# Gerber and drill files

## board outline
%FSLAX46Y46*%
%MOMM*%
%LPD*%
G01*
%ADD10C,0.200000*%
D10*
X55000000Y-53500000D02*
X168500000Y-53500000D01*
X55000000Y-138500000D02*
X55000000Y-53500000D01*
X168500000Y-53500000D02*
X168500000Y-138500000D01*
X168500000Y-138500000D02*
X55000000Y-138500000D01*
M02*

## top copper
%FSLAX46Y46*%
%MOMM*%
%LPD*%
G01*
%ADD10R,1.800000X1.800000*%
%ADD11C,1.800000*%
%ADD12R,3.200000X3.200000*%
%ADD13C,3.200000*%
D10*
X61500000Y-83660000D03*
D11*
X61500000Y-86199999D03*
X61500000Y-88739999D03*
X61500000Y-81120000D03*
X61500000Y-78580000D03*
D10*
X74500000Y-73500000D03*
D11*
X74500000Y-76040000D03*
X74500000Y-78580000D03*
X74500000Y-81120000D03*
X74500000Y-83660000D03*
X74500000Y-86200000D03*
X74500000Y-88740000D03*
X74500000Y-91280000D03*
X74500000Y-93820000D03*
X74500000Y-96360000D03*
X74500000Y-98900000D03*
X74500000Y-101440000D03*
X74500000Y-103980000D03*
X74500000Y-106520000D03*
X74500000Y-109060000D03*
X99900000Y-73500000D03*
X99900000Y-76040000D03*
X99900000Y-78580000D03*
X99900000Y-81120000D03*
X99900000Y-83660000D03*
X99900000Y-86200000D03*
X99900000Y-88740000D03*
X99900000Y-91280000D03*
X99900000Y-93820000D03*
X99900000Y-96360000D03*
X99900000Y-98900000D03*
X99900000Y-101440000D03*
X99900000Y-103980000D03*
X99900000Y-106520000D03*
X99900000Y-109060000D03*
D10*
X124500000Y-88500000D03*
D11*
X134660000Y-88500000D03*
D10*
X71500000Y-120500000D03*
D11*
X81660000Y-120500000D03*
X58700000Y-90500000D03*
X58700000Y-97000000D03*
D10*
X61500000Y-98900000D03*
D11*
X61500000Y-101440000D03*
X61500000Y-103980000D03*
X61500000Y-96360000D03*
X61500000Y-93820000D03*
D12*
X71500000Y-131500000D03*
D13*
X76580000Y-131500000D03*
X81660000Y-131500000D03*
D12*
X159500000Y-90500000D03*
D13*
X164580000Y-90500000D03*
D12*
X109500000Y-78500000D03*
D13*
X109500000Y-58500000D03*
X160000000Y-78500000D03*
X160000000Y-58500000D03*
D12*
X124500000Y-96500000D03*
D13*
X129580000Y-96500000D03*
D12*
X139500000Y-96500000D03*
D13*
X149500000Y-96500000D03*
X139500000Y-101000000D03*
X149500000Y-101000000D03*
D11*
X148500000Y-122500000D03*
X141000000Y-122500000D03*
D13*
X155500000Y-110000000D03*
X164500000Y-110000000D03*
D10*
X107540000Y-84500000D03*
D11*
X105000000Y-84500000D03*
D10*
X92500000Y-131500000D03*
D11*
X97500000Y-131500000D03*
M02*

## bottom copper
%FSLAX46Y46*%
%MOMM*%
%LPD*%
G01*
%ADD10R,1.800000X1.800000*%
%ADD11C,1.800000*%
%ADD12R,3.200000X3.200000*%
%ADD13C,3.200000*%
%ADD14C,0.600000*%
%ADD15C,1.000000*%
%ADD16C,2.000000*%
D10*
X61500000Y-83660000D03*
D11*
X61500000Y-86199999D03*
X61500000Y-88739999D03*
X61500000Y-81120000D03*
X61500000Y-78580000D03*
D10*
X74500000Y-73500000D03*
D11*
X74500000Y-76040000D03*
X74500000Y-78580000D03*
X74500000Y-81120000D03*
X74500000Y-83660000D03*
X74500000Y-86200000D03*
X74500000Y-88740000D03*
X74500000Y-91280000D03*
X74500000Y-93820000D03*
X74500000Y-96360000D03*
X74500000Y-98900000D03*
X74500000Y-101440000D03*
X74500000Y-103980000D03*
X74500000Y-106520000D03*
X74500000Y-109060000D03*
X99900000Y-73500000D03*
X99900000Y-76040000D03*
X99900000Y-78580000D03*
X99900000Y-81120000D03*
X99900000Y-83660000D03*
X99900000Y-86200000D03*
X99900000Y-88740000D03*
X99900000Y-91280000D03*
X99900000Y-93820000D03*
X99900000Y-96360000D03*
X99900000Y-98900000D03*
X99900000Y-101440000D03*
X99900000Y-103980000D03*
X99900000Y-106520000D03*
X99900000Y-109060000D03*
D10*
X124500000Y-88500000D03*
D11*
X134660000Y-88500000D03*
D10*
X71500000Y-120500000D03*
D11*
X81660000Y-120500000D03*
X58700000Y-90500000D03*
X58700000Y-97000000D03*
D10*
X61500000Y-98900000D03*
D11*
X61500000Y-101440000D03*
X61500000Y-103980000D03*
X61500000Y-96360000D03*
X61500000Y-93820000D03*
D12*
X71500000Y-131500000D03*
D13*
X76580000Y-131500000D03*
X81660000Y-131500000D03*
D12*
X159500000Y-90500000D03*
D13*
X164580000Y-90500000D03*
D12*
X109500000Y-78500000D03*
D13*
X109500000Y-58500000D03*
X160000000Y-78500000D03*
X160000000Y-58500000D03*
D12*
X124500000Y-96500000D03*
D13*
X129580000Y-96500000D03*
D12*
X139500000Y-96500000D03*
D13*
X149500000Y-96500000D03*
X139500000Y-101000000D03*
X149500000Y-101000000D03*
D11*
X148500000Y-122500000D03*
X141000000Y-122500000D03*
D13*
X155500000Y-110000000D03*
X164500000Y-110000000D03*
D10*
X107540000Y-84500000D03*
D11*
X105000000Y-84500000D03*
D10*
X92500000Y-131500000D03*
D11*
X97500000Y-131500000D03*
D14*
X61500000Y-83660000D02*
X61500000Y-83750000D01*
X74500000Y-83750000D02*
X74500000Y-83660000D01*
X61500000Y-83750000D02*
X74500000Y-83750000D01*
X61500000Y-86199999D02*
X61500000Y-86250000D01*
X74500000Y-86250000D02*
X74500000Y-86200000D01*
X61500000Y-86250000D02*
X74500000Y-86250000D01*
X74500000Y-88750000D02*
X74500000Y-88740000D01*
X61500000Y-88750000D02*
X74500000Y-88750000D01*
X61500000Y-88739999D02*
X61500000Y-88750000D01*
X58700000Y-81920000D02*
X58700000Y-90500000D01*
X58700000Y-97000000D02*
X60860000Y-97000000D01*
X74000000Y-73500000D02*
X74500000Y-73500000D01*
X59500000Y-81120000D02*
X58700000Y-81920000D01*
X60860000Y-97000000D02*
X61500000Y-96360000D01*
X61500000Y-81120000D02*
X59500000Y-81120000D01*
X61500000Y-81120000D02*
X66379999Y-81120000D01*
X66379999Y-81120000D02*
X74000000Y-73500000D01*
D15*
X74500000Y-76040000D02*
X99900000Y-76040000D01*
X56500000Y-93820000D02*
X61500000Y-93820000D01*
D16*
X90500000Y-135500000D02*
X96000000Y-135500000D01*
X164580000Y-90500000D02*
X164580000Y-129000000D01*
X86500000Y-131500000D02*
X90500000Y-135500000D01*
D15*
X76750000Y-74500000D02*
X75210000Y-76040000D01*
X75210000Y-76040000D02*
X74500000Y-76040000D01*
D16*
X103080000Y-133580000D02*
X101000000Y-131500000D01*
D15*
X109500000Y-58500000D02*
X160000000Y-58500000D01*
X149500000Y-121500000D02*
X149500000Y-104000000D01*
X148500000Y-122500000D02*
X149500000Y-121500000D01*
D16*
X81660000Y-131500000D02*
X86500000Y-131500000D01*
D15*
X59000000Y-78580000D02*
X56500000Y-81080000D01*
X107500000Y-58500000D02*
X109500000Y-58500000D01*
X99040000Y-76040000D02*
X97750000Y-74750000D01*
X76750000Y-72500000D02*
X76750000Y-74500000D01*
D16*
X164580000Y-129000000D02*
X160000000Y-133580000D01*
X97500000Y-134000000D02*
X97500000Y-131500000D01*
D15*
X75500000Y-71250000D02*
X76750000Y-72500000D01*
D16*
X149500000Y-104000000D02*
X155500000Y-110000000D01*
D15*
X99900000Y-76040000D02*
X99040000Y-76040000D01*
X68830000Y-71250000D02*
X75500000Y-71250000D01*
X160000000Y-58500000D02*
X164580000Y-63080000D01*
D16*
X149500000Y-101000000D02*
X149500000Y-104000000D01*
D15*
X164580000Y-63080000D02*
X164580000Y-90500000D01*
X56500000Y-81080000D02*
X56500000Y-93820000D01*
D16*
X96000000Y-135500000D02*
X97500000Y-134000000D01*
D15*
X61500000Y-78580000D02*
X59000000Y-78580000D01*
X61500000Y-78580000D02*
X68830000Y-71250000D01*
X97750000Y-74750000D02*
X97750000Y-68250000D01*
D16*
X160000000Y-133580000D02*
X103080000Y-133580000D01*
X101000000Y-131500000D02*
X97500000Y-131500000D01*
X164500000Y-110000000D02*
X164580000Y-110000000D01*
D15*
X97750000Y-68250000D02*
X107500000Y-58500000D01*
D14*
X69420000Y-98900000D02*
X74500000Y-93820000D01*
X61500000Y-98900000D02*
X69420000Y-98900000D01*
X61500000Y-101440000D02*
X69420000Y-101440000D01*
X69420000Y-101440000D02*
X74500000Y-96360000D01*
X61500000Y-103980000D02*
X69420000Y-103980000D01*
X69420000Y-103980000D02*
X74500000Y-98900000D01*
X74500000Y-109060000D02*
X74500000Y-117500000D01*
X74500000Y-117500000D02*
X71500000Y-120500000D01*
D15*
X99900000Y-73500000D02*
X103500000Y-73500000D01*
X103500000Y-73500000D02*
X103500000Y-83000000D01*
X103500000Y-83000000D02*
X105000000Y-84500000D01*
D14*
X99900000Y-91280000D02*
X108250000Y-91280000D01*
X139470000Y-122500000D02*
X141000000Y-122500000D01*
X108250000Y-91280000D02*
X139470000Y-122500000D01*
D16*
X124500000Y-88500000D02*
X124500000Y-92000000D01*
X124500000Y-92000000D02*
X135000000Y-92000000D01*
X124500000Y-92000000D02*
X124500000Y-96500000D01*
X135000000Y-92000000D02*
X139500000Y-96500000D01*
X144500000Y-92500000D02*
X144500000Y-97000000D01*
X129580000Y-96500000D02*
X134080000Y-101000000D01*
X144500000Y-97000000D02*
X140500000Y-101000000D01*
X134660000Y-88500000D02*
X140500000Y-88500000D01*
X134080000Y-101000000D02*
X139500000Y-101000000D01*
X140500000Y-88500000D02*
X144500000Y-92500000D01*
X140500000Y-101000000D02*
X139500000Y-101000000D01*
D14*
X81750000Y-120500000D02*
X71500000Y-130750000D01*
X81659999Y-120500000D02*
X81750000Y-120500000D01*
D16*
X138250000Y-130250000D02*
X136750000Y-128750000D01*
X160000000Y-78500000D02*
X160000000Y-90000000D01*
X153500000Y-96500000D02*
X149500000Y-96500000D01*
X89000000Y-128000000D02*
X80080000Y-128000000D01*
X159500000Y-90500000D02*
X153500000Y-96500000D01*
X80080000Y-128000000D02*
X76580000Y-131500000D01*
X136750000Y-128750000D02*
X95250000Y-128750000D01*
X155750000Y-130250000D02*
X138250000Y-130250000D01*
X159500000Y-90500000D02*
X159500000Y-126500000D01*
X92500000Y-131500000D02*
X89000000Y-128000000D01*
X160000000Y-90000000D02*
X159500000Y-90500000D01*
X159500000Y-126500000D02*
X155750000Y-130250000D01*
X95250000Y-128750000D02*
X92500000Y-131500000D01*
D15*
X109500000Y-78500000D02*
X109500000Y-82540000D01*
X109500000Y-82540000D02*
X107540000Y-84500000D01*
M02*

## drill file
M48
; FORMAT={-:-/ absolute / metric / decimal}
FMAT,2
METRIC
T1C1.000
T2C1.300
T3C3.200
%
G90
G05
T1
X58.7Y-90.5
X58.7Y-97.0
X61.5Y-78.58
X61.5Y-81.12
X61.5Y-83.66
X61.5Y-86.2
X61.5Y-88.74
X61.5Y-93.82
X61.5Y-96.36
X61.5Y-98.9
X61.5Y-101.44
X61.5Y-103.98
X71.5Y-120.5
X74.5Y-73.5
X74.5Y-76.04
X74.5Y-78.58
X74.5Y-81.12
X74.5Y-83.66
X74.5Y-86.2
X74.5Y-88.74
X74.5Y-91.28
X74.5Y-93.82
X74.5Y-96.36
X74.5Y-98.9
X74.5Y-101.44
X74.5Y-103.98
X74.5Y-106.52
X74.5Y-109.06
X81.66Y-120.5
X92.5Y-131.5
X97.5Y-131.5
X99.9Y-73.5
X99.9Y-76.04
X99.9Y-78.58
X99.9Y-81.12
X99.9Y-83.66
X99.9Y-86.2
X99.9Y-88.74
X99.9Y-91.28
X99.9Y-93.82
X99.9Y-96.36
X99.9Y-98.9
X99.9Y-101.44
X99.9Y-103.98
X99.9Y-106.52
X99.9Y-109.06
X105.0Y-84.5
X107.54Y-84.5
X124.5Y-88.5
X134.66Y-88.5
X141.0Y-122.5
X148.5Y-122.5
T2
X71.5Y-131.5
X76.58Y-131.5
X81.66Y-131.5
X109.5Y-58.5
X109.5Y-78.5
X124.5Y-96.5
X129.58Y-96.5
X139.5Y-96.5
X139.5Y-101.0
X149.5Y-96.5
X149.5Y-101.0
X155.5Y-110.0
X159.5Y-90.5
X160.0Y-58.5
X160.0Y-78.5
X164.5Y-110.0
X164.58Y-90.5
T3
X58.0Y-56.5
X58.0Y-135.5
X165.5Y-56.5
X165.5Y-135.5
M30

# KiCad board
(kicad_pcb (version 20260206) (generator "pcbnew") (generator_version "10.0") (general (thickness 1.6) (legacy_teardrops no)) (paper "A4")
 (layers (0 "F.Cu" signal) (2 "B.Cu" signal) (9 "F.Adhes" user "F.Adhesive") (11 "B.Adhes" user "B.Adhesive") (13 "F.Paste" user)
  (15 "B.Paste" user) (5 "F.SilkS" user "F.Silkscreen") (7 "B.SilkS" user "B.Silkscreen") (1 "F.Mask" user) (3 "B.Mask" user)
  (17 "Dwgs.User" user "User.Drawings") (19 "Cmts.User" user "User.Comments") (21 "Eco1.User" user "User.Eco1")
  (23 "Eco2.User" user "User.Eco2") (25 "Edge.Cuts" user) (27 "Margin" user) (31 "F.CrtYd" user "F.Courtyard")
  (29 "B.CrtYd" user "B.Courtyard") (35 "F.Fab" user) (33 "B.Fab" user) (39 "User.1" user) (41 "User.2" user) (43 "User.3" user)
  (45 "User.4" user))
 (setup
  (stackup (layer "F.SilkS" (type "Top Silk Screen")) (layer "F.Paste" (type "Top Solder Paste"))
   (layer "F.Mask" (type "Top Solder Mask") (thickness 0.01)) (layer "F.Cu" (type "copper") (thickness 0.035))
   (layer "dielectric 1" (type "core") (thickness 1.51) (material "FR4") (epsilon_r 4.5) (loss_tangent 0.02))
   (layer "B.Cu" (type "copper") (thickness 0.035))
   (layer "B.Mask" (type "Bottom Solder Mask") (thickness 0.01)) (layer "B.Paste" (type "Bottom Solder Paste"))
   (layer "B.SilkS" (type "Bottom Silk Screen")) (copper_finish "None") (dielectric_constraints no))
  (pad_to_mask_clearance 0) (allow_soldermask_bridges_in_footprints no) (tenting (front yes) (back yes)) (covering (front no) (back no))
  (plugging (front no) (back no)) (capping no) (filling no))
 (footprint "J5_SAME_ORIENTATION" (layer "F.Cu") (at 61.5 83.5 -90)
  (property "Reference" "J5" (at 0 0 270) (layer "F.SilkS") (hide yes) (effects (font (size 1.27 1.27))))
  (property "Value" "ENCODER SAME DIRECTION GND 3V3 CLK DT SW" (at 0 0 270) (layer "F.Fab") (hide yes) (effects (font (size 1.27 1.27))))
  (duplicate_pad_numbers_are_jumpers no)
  (pad "1" thru_hole rect (at 0.16 0 270) (size 1.8 1.8) (drill 1) (layers "*.Cu") (remove_unused_layers no) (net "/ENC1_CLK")
   (clearance 0.5) (thermal_bridge_angle 45))
  (pad "2" thru_hole circle (at 2.699999 0 270) (size 1.8 1.8) (drill 1) (layers "*.Cu") (remove_unused_layers no) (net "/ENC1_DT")
   (clearance 0.5))
  (pad "3" thru_hole circle (at 5.239999 0 270) (size 1.8 1.8) (drill 1) (layers "*.Cu") (remove_unused_layers no) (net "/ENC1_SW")
   (clearance 0.5))
  (pad "4" thru_hole circle (at -2.38 0 270) (size 1.8 1.8) (drill 1) (layers "*.Cu") (remove_unused_layers no) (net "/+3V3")
   (clearance 0.5))
  (pad "5" thru_hole circle (at -4.92 0 270) (size 1.8 1.8) (drill 1) (layers "*.Cu") (remove_unused_layers no) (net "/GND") (clearance 0.5)))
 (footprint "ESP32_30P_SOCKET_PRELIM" (layer "F.Cu") (at 74.5 73.5)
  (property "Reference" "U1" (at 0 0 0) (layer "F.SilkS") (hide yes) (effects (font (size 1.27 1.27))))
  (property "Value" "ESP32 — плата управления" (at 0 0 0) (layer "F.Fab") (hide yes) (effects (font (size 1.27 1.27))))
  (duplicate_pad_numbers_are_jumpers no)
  (pad "1" thru_hole rect (at 0 0) (size 1.8 1.8) (drill 1) (layers "*.Cu") (remove_unused_layers no) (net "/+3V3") (clearance 0.5)
   (thermal_bridge_angle 45))
  (pad "2" thru_hole circle (at 0 2.54) (size 1.8 1.8) (drill 1) (layers "*.Cu") (remove_unused_layers no) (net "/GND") (clearance 0.5))
  (pad "3" thru_hole circle (at 0 5.08) (size 1.8 1.8) (drill 1) (layers "*.Cu") (remove_unused_layers no) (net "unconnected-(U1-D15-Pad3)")
   (clearance 0.5))
  (pad "4" thru_hole circle (at 0 7.62) (size 1.8 1.8) (drill 1) (layers "*.Cu") (remove_unused_layers no) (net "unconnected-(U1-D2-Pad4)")
   (clearance 0.5))
  (pad "5" thru_hole circle (at 0 10.16) (size 1.8 1.8) (drill 1) (layers "*.Cu") (remove_unused_layers no) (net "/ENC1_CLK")
   (clearance 0.5))
  (pad "6" thru_hole circle (at 0 12.7) (size 1.8 1.8) (drill 1) (layers "*.Cu") (remove_unused_layers no) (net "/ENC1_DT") (clearance 0.5))
  (pad "7" thru_hole circle (at 0 15.24) (size 1.8 1.8) (drill 1) (layers "*.Cu") (remove_unused_layers no) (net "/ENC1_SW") (clearance 0.5))
  (pad "8" thru_hole circle (at 0 17.78) (size 1.8 1.8) (drill 1) (layers "*.Cu") (remove_unused_layers no) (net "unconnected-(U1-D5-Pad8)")
   (clearance 0.5))
  (pad "9" thru_hole circle (at 0 20.32) (size 1.8 1.8) (drill 1) (layers "*.Cu") (remove_unused_layers no) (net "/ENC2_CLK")
   (clearance 0.5))
  (pad "10" thru_hole circle (at 0 22.86) (size 1.8 1.8) (drill 1) (layers "*.Cu") (remove_unused_layers no) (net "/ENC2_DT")
   (clearance 0.5))
  (pad "11" thru_hole circle (at 0 25.4) (size 1.8 1.8) (drill 1) (layers "*.Cu") (remove_unused_layers no) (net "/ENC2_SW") (clearance 0.5))
  (pad "12" thru_hole circle (at 0 27.94) (size 1.8 1.8) (drill 1) (layers "*.Cu") (remove_unused_layers no)
   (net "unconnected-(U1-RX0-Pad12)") (clearance 0.5))
  (pad "13" thru_hole circle (at 0 30.48) (size 1.8 1.8) (drill 1) (layers "*.Cu") (remove_unused_layers no)
   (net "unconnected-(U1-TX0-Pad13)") (clearance 0.5))
  (pad "14" thru_hole circle (at 0 33.02) (size 1.8 1.8) (drill 1) (layers "*.Cu") (remove_unused_layers no)
   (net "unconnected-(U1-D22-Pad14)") (clearance 0.5))
  (pad "15" thru_hole circle (at 0 35.56) (size 1.8 1.8) (drill 1) (layers "*.Cu") (remove_unused_layers no) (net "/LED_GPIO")
   (clearance 0.5))
  (pad "16" thru_hole circle (at 25.4 0) (size 1.8 1.8) (drill 1) (layers "*.Cu") (remove_unused_layers no) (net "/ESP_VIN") (clearance 0.5))
  (pad "17" thru_hole circle (at 25.4 2.54) (size 1.8 1.8) (drill 1) (layers "*.Cu") (remove_unused_layers no) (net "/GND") (clearance 0.5))
  (pad "18" thru_hole circle (at 25.4 5.08) (size 1.8 1.8) (drill 1) (layers "*.Cu") (remove_unused_layers no)
   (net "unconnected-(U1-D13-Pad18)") (clearance 0.5))
  (pad "19" thru_hole circle (at 25.4 7.62) (size 1.8 1.8) (drill 1) (layers "*.Cu") (remove_unused_layers no)
   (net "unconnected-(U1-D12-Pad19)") (clearance 0.5))
  (pad "20" thru_hole circle (at 25.4 10.16) (size 1.8 1.8) (drill 1) (layers "*.Cu") (remove_unused_layers no)
   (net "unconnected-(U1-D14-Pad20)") (clearance 0.5))
  (pad "21" thru_hole circle (at 25.4 12.7) (size 1.8 1.8) (drill 1) (layers "*.Cu") (remove_unused_layers no)
   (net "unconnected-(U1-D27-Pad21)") (clearance 0.5))
  (pad "22" thru_hole circle (at 25.4 15.24) (size 1.8 1.8) (drill 1) (layers "*.Cu") (remove_unused_layers no)
   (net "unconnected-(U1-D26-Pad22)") (clearance 0.5))
  (pad "23" thru_hole circle (at 25.4 17.78) (size 1.8 1.8) (drill 1) (layers "*.Cu") (remove_unused_layers no) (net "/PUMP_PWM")
   (clearance 0.5))
  (pad "24" thru_hole circle (at 25.4 20.32) (size 1.8 1.8) (drill 1) (layers "*.Cu") (remove_unused_layers no)
   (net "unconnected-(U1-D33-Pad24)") (clearance 0.5))
  (pad "25" thru_hole circle (at 25.4 22.86) (size 1.8 1.8) (drill 1) (layers "*.Cu") (remove_unused_layers no)
   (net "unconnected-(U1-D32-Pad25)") (clearance 0.5))
  (pad "26" thru_hole circle (at 25.4 25.4) (size 1.8 1.8) (drill 1) (layers "*.Cu") (remove_unused_layers no)
   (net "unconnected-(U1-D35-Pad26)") (clearance 0.5))
  (pad "27" thru_hole circle (at 25.4 27.94) (size 1.8 1.8) (drill 1) (layers "*.Cu") (remove_unused_layers no)
   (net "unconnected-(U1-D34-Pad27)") (clearance 0.5))
  (pad "28" thru_hole circle (at 25.4 30.48) (size 1.8 1.8) (drill 1) (layers "*.Cu") (remove_unused_layers no)
   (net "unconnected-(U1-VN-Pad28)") (clearance 0.5))
  (pad "29" thru_hole circle (at 25.4 33.02) (size 1.8 1.8) (drill 1) (layers "*.Cu") (remove_unused_layers no)
   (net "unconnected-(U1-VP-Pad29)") (clearance 0.5))
  (pad "30" thru_hole circle (at 25.4 35.56) (size 1.8 1.8) (drill 1) (layers "*.Cu") (remove_unused_layers no)
   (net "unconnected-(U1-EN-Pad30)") (clearance 0.5)))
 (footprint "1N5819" (layer "F.Cu") (at 124.5 88.5)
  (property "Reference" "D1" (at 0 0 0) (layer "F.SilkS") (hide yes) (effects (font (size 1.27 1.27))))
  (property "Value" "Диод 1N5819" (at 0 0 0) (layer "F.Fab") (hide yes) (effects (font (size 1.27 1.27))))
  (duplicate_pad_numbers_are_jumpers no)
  (pad "1" thru_hole rect (at 0 0) (size 1.8 1.8) (drill 1) (layers "*.Cu") (remove_unused_layers no) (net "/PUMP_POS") (clearance 0.5)
   (thermal_bridge_angle 45))
  (pad "2" thru_hole circle (at 10.16 0) (size 1.8 1.8) (drill 1) (layers "*.Cu") (remove_unused_layers no) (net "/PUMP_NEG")
   (clearance 0.5)))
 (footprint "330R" (layer "F.Cu") (at 71.5 120.5)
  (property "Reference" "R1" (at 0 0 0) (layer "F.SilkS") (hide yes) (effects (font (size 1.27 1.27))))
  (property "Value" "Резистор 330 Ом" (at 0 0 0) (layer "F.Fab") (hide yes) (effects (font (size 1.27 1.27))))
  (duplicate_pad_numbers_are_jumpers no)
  (pad "1" thru_hole rect (at 0 0) (size 1.8 1.8) (drill 1) (layers "*.Cu") (remove_unused_layers no) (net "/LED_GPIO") (clearance 0.5)
   (thermal_bridge_angle 45))
  (pad "2" thru_hole circle (at 10.16 0) (size 1.8 1.8) (drill 1) (layers "*.Cu") (remove_unused_layers no) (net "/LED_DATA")
   (clearance 0.5)))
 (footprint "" (layer "F.Cu") (at 58 135.5)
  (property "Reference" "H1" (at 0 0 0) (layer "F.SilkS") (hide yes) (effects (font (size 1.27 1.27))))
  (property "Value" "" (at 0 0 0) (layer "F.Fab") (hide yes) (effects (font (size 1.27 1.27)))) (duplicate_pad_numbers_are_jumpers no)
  (pad "" np_thru_hole circle (at 0 0) (size 3.2 3.2) (drill 3.2) (layers "*.Cu") (clearance 0.5)))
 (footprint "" (layer "F.Cu") (at 58.7 90.5)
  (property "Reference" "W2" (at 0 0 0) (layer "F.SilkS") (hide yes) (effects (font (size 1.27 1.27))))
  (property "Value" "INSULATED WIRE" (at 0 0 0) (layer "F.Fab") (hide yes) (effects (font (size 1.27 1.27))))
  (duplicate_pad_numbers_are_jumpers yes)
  (pad "1" thru_hole circle (at 0 0) (size 1.8 1.8) (drill 1) (layers "*.Cu") (remove_unused_layers no) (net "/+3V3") (clearance 0.5))
  (pad "1" thru_hole circle (at 0 6.5) (size 1.8 1.8) (drill 1) (layers "*.Cu") (remove_unused_layers no) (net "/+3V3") (clearance 0.5)))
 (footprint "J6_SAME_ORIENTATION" (layer "F.Cu") (at 61.5 96.5 -90)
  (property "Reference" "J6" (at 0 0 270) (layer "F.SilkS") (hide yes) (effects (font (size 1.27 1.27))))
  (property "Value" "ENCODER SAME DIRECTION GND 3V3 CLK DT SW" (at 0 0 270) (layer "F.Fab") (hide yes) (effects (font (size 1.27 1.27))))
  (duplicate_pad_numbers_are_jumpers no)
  (pad "1" thru_hole rect (at 2.4 0 270) (size 1.8 1.8) (drill 1) (layers "*.Cu") (remove_unused_layers no) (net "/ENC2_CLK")
   (clearance 0.5) (thermal_bridge_angle 45))
  (pad "2" thru_hole circle (at 4.94 0 270) (size 1.8 1.8) (drill 1) (layers "*.Cu") (remove_unused_layers no) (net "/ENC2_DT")
   (clearance 0.5))
  (pad "3" thru_hole circle (at 7.48 0 270) (size 1.8 1.8) (drill 1) (layers "*.Cu") (remove_unused_layers no) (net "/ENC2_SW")
   (clearance 0.5))
  (pad "4" thru_hole circle (at -0.14 0 270) (size 1.8 1.8) (drill 1) (layers "*.Cu") (remove_unused_layers no) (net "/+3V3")
   (clearance 0.5))
  (pad "5" thru_hole circle (at -2.68 0 270) (size 1.8 1.8) (drill 1) (layers "*.Cu") (remove_unused_layers no) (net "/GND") (clearance 0.5)))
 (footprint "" (layer "F.Cu") (at 58 56.5)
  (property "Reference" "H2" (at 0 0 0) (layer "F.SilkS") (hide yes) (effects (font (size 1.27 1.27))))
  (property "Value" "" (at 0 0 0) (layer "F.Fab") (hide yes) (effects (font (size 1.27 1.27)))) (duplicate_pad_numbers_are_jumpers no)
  (pad "" np_thru_hole circle (at 0 0) (size 3.2 3.2) (drill 3.2) (layers "*.Cu") (clearance 0.5)))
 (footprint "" (layer "F.Cu") (at 165.5 135.5)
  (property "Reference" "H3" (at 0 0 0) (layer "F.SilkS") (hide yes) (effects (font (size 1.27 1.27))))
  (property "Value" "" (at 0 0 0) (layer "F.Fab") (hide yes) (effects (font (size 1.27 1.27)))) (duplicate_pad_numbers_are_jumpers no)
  (pad "" np_thru_hole circle (at 0 0) (size 3.2 3.2) (drill 3.2) (layers "*.Cu") (clearance 0.5)))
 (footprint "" (layer "F.Cu") (at 165.5 56.5)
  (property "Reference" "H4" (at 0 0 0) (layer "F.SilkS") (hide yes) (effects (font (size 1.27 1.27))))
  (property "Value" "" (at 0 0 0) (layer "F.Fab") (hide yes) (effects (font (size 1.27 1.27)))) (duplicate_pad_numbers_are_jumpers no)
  (pad "" np_thru_hole circle (at 0 0) (size 3.2 3.2) (drill 3.2) (layers "*.Cu") (clearance 0.5)))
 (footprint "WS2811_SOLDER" (layer "F.Cu") (at 71.5 131.5)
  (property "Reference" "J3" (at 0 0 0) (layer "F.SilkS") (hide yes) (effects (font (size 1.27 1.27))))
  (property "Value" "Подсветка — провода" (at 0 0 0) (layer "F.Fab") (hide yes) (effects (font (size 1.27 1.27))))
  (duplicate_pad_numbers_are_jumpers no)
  (pad "1" thru_hole rect (at 0 0) (size 3.2 3.2) (drill 1.3) (layers "*.Cu") (remove_unused_layers no) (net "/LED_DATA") (clearance 0.5)
   (thermal_bridge_angle 45))
  (pad "2" thru_hole circle (at 5.08 0) (size 3.2 3.2) (drill 1.3) (layers "*.Cu") (remove_unused_layers no) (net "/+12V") (clearance 0.5))
  (pad "3" thru_hole circle (at 10.16 0) (size 3.2 3.2) (drill 1.3) (layers "*.Cu") (remove_unused_layers no) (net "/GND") (clearance 0.5)))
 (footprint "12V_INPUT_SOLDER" (layer "F.Cu") (at 159.5 90.5)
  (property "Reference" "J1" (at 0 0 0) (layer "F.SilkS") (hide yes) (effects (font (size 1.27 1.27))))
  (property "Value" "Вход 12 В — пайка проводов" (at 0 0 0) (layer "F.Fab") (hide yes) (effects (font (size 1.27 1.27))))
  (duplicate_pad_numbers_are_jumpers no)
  (pad "1" thru_hole rect (at 0 0) (size 3.2 3.2) (drill 1.3) (layers "*.Cu") (remove_unused_layers no) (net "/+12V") (clearance 0.5)
   (thermal_bridge_angle 45))
  (pad "2" thru_hole circle (at 5.08 0) (size 3.2 3.2) (drill 1.3) (layers "*.Cu") (remove_unused_layers no) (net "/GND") (clearance 0.5)))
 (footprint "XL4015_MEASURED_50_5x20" (layer "F.Cu") (at 109.5 78.5 90)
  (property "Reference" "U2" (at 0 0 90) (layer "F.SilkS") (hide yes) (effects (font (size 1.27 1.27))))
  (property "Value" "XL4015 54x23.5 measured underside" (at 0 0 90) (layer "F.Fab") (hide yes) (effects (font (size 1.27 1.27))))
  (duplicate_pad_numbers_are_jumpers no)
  (pad "1" thru_hole rect (at 0 0 90) (size 3.2 3.2) (drill 1.3) (layers "*.Cu") (remove_unused_layers no) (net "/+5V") (clearance 0.5)
   (thermal_bridge_angle 45))
  (pad "2" thru_hole circle (at 20 0 90) (size 3.2 3.2) (drill 1.3) (layers "*.Cu") (remove_unused_layers no) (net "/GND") (clearance 0.5))
  (pad "3" thru_hole circle (at 0 50.5 90) (size 3.2 3.2) (drill 1.3) (layers "*.Cu") (remove_unused_layers no) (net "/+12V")
   (clearance 0.5))
  (pad "4" thru_hole circle (at 20 50.5 90) (size 3.2 3.2) (drill 1.3) (layers "*.Cu") (remove_unused_layers no) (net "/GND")
   (clearance 0.5)))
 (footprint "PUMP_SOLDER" (layer "F.Cu") (at 124.5 96.5)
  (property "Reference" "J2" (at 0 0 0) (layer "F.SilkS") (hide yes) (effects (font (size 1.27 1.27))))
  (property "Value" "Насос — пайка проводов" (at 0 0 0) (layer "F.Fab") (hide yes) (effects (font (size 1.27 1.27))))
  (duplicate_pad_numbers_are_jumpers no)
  (pad "1" thru_hole rect (at 0 0) (size 3.2 3.2) (drill 1.3) (layers "*.Cu") (remove_unused_layers no) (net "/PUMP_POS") (clearance 0.5)
   (thermal_bridge_angle 45))
  (pad "2" thru_hole circle (at 5.08 0) (size 3.2 3.2) (drill 1.3) (layers "*.Cu") (remove_unused_layers no) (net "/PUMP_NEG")
   (clearance 0.5)))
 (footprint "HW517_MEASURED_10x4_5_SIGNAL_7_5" (layer "F.Cu") (at 139.5 96.5)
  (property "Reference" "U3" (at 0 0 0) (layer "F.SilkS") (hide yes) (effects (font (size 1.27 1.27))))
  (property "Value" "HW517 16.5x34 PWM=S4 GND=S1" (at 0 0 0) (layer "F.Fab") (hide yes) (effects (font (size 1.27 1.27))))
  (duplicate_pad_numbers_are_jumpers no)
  (pad "1" thru_hole rect (at 0 0) (size 3.2 3.2) (drill 1.3) (layers "*.Cu") (remove_unused_layers no) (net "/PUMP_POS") (clearance 0.5)
   (thermal_bridge_angle 45))
  (pad "2" thru_hole circle (at 10 0) (size 3.2 3.2) (drill 1.3) (layers "*.Cu") (remove_unused_layers no) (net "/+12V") (clearance 0.5))
  (pad "3" thru_hole circle (at 0 4.5) (size 3.2 3.2) (drill 1.3) (layers "*.Cu") (remove_unused_layers no) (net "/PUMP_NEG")
   (clearance 0.5))
  (pad "4" thru_hole circle (at 10 4.5) (size 3.2 3.2) (drill 1.3) (layers "*.Cu") (remove_unused_layers no) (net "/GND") (clearance 0.5))
  (pad "5" thru_hole circle (at 9 26) (size 1.8 1.8) (drill 1) (layers "*.Cu") (remove_unused_layers no) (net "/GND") (clearance 0.5))
  (pad "6" thru_hole circle (at 1.5 26) (size 1.8 1.8) (drill 1) (layers "*.Cu") (remove_unused_layers no) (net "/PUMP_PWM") (clearance 0.5)))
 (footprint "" (layer "F.Cu") (at 155.5 110)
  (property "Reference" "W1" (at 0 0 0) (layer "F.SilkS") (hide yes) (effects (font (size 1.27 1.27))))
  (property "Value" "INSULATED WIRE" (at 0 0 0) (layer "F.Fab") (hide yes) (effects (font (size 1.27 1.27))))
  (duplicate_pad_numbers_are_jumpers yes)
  (pad "1" thru_hole circle (at 0 0) (size 3.2 3.2) (drill 1.3) (layers "*.Cu") (remove_unused_layers no) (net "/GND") (clearance 0.5))
  (pad "1" thru_hole circle (at 9 0) (size 3.2 3.2) (drill 1.3) (layers "*.Cu") (remove_unused_layers no) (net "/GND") (clearance 0.5)))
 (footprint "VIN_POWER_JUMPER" (layer "F.Cu") (at 107.54 84.5)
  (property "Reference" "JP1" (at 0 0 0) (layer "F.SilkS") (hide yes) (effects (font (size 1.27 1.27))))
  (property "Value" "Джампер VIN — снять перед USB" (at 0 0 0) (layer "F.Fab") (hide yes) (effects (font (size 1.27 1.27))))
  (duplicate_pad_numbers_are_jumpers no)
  (pad "1" thru_hole rect (at 0 0) (size 1.8 1.8) (drill 1) (layers "*.Cu") (remove_unused_layers no) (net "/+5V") (clearance 0.5)
   (thermal_bridge_angle 45))
  (pad "2" thru_hole circle (at -2.54 0) (size 1.8 1.8) (drill 1) (layers "*.Cu") (remove_unused_layers no) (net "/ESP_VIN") (clearance 0.5)))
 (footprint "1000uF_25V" (layer "F.Cu") (at 92.5 131.5)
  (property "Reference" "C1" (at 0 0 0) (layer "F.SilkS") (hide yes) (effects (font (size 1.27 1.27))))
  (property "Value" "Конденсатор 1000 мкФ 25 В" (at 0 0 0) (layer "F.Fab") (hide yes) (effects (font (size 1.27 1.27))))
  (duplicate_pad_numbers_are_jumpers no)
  (pad "1" thru_hole rect (at 0 0) (size 1.8 1.8) (drill 1) (layers "*.Cu") (remove_unused_layers no) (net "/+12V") (clearance 0.5)
   (thermal_bridge_angle 45))
  (pad "2" thru_hole circle (at 5 0) (size 1.8 1.8) (drill 1) (layers "*.Cu") (remove_unused_layers no) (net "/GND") (clearance 0.5)))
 (gr_line (start 55 53.5) (end 168.5 53.5) (stroke (width 0.2) (type default)) (layer "Edge.Cuts"))
 (gr_line (start 55 138.5) (end 55 53.5) (stroke (width 0.2) (type default)) (layer "Edge.Cuts"))
 (gr_line (start 168.5 53.5) (end 168.5 138.5) (stroke (width 0.2) (type default)) (layer "Edge.Cuts"))
 (gr_line (start 168.5 138.5) (end 55 138.5) (stroke (width 0.2) (type default)) (layer "Edge.Cuts"))
 (segment (start 61.5 83.66) (end 61.5 83.75) (width 0.6) (layer "B.Cu") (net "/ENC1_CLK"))
 (segment (start 74.5 83.75) (end 74.5 83.66) (width 0.6) (layer "B.Cu") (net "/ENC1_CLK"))
 (segment (start 61.5 83.75) (end 74.5 83.75) (width 0.6) (layer "B.Cu") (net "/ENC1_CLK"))
 (segment (start 61.5 86.199999) (end 61.5 86.25) (width 0.6) (layer "B.Cu") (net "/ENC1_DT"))
 (segment (start 74.5 86.25) (end 74.5 86.2) (width 0.6) (layer "B.Cu") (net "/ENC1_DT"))
 (segment (start 61.5 86.25) (end 74.5 86.25) (width 0.6) (layer "B.Cu") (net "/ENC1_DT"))
 (segment (start 74.5 88.75) (end 74.5 88.74) (width 0.6) (layer "B.Cu") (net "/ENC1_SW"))
 (segment (start 61.5 88.75) (end 74.5 88.75) (width 0.6) (layer "B.Cu") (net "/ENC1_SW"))
 (segment (start 61.5 88.739999) (end 61.5 88.75) (width 0.6) (layer "B.Cu") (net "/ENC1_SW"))
 (segment (start 58.7 81.92) (end 58.7 90.5) (width 0.6) (layer "B.Cu") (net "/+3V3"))
 (segment (start 58.7 97) (end 60.86 97) (width 0.6) (layer "B.Cu") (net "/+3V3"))
 (segment (start 74 73.5) (end 74.5 73.5) (width 0.6) (layer "B.Cu") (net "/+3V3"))
 (segment (start 59.5 81.12) (end 58.7 81.92) (width 0.6) (layer "B.Cu") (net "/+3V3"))
 (segment (start 60.86 97) (end 61.5 96.36) (width 0.6) (layer "B.Cu") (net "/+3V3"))
 (segment (start 61.5 81.12) (end 59.5 81.12) (width 0.6) (layer "B.Cu") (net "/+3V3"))
 (segment (start 61.5 81.12) (end 66.379999 81.12) (width 0.6) (layer "B.Cu") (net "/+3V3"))
 (segment (start 66.379999 81.12) (end 74 73.5) (width 0.6) (layer "B.Cu") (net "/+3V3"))
 (segment (start 74.5 76.04) (end 99.9 76.04) (width 1) (layer "B.Cu") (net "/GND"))
 (segment (start 56.5 93.82) (end 61.5 93.82) (width 1) (layer "B.Cu") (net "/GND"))
 (segment (start 90.5 135.5) (end 96 135.5) (width 2) (layer "B.Cu") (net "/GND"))
 (segment (start 164.58 90.5) (end 164.58 129) (width 2) (layer "B.Cu") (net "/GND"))
 (segment (start 86.5 131.5) (end 90.5 135.5) (width 2) (layer "B.Cu") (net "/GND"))
 (segment (start 76.75 74.5) (end 75.21 76.04) (width 1) (layer "B.Cu") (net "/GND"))
 (segment (start 75.21 76.04) (end 74.5 76.04) (width 1) (layer "B.Cu") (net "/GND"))
 (segment (start 103.08 133.58) (end 101 131.5) (width 2) (layer "B.Cu") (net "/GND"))
 (segment (start 109.5 58.5) (end 160 58.5) (width 1) (layer "B.Cu") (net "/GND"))
 (segment (start 149.5 121.5) (end 149.5 104) (width 1) (layer "B.Cu") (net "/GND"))
 (segment (start 148.5 122.5) (end 149.5 121.5) (width 1) (layer "B.Cu") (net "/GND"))
 (segment (start 81.66 131.5) (end 86.5 131.5) (width 2) (layer "B.Cu") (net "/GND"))
 (segment (start 59 78.58) (end 56.5 81.08) (width 1) (layer "B.Cu") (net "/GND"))
 (segment (start 107.5 58.5) (end 109.5 58.5) (width 1) (layer "B.Cu") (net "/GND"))
 (segment (start 99.04 76.04) (end 97.75 74.75) (width 1) (layer "B.Cu") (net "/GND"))
 (segment (start 76.75 72.5) (end 76.75 74.5) (width 1) (layer "B.Cu") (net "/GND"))
 (segment (start 164.58 129) (end 160 133.58) (width 2) (layer "B.Cu") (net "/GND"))
 (segment (start 97.5 134) (end 97.5 131.5) (width 2) (layer "B.Cu") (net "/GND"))
 (segment (start 75.5 71.25) (end 76.75 72.5) (width 1) (layer "B.Cu") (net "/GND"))
 (segment (start 149.5 104) (end 155.5 110) (width 2) (layer "B.Cu") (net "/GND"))
 (segment (start 99.9 76.04) (end 99.04 76.04) (width 1) (layer "B.Cu") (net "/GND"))
 (segment (start 68.83 71.25) (end 75.5 71.25) (width 1) (layer "B.Cu") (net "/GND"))
 (segment (start 160 58.5) (end 164.58 63.08) (width 1) (layer "B.Cu") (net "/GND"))
 (segment (start 149.5 101) (end 149.5 104) (width 2) (layer "B.Cu") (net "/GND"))
 (segment (start 164.58 63.08) (end 164.58 90.5) (width 1) (layer "B.Cu") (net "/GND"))
 (segment (start 56.5 81.08) (end 56.5 93.82) (width 1) (layer "B.Cu") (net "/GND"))
 (segment (start 96 135.5) (end 97.5 134) (width 2) (layer "B.Cu") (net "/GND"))
 (segment (start 61.5 78.58) (end 59 78.58) (width 1) (layer "B.Cu") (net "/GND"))
 (segment (start 61.5 78.58) (end 68.83 71.25) (width 1) (layer "B.Cu") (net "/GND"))
 (segment (start 97.75 74.75) (end 97.75 68.25) (width 1) (layer "B.Cu") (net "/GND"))
 (segment (start 160 133.58) (end 103.08 133.58) (width 2) (layer "B.Cu") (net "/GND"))
 (segment (start 101 131.5) (end 97.5 131.5) (width 2) (layer "B.Cu") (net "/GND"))
 (segment (start 164.5 110) (end 164.58 110) (width 2) (layer "B.Cu") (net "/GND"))
 (segment (start 97.75 68.25) (end 107.5 58.5) (width 1) (layer "B.Cu") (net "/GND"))
 (segment (start 69.42 98.9) (end 74.5 93.82) (width 0.6) (layer "B.Cu") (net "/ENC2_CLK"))
 (segment (start 61.5 98.9) (end 69.42 98.9) (width 0.6) (layer "B.Cu") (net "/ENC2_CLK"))
 (segment (start 61.5 101.44) (end 69.42 101.44) (width 0.6) (layer "B.Cu") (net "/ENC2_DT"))
 (segment (start 69.42 101.44) (end 74.5 96.36) (width 0.6) (layer "B.Cu") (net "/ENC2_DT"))
 (segment (start 61.5 103.98) (end 69.42 103.98) (width 0.6) (layer "B.Cu") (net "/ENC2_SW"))
 (segment (start 69.42 103.98) (end 74.5 98.9) (width 0.6) (layer "B.Cu") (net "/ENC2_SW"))
 (segment (start 74.5 109.06) (end 74.5 117.5) (width 0.6) (layer "B.Cu") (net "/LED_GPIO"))
 (segment (start 74.5 117.5) (end 71.5 120.5) (width 0.6) (layer "B.Cu") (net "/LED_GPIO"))
 (segment (start 99.9 73.5) (end 103.5 73.5) (width 1) (layer "B.Cu") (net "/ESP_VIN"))
 (segment (start 103.5 73.5) (end 103.5 83) (width 1) (layer "B.Cu") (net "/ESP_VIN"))
 (segment (start 103.5 83) (end 105 84.5) (width 1) (layer "B.Cu") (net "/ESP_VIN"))
 (segment (start 99.9 91.28) (end 108.25 91.28) (width 0.6) (layer "B.Cu") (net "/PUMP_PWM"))
 (segment (start 139.47 122.5) (end 141 122.5) (width 0.6) (layer "B.Cu") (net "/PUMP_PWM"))
 (segment (start 108.25 91.28) (end 139.47 122.5) (width 0.6) (layer "B.Cu") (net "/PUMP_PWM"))
 (segment (start 124.5 88.5) (end 124.5 92) (width 2) (layer "B.Cu") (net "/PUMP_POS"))
 (segment (start 124.5 92) (end 135 92) (width 2) (layer "B.Cu") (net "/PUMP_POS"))
 (segment (start 124.5 92) (end 124.5 96.5) (width 2) (layer "B.Cu") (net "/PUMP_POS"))
 (segment (start 135 92) (end 139.5 96.5) (width 2) (layer "B.Cu") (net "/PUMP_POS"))
 (segment (start 144.5 92.5) (end 144.5 97) (width 2) (layer "B.Cu") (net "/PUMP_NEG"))
 (segment (start 129.58 96.5) (end 134.08 101) (width 2) (layer "B.Cu") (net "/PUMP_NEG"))
 (segment (start 144.5 97) (end 140.5 101) (width 2) (layer "B.Cu") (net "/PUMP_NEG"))
 (segment (start 134.66 88.5) (end 140.5 88.5) (width 2) (layer "B.Cu") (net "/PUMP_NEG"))
 (segment (start 134.08 101) (end 139.5 101) (width 2) (layer "B.Cu") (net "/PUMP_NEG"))
 (segment (start 140.5 88.5) (end 144.5 92.5) (width 2) (layer "B.Cu") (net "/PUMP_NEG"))
 (segment (start 140.5 101) (end 139.5 101) (width 2) (layer "B.Cu") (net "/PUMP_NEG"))
 (segment (start 81.75 120.5) (end 71.5 130.75) (width 0.6) (layer "B.Cu") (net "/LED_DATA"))
 (segment (start 81.659999 120.5) (end 81.75 120.5) (width 0.6) (layer "B.Cu") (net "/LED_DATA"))
 (segment (start 138.25 130.25) (end 136.75 128.75) (width 2) (layer "B.Cu") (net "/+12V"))
 (segment (start 160 78.5) (end 160 90) (width 2) (layer "B.Cu") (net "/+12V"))
 (segment (start 153.5 96.5) (end 149.5 96.5) (width 2) (layer "B.Cu") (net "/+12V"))
 (segment (start 89 128) (end 80.08 128) (width 2) (layer "B.Cu") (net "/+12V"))
 (segment (start 159.5 90.5) (end 153.5 96.5) (width 2) (layer "B.Cu") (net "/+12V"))
 (segment (start 80.08 128) (end 76.58 131.5) (width 2) (layer "B.Cu") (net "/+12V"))
 (segment (start 136.75 128.75) (end 95.25 128.75) (width 2) (layer "B.Cu") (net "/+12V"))
 (segment (start 155.75 130.25) (end 138.25 130.25) (width 2) (layer "B.Cu") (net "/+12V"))
 (segment (start 159.5 90.5) (end 159.5 126.5) (width 2) (layer "B.Cu") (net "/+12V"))
 (segment (start 92.5 131.5) (end 89 128) (width 2) (layer "B.Cu") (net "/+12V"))
 (segment (start 160 90) (end 159.5 90.5) (width 2) (layer "B.Cu") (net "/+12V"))
 (segment (start 159.5 126.5) (end 155.75 130.25) (width 2) (layer "B.Cu") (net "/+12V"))
 (segment (start 95.25 128.75) (end 92.5 131.5) (width 2) (layer "B.Cu") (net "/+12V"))
 (segment (start 109.5 78.5) (end 109.5 82.54) (width 1) (layer "B.Cu") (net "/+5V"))
 (segment (start 109.5 82.54) (end 107.54 84.5) (width 1) (layer "B.Cu") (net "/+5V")))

